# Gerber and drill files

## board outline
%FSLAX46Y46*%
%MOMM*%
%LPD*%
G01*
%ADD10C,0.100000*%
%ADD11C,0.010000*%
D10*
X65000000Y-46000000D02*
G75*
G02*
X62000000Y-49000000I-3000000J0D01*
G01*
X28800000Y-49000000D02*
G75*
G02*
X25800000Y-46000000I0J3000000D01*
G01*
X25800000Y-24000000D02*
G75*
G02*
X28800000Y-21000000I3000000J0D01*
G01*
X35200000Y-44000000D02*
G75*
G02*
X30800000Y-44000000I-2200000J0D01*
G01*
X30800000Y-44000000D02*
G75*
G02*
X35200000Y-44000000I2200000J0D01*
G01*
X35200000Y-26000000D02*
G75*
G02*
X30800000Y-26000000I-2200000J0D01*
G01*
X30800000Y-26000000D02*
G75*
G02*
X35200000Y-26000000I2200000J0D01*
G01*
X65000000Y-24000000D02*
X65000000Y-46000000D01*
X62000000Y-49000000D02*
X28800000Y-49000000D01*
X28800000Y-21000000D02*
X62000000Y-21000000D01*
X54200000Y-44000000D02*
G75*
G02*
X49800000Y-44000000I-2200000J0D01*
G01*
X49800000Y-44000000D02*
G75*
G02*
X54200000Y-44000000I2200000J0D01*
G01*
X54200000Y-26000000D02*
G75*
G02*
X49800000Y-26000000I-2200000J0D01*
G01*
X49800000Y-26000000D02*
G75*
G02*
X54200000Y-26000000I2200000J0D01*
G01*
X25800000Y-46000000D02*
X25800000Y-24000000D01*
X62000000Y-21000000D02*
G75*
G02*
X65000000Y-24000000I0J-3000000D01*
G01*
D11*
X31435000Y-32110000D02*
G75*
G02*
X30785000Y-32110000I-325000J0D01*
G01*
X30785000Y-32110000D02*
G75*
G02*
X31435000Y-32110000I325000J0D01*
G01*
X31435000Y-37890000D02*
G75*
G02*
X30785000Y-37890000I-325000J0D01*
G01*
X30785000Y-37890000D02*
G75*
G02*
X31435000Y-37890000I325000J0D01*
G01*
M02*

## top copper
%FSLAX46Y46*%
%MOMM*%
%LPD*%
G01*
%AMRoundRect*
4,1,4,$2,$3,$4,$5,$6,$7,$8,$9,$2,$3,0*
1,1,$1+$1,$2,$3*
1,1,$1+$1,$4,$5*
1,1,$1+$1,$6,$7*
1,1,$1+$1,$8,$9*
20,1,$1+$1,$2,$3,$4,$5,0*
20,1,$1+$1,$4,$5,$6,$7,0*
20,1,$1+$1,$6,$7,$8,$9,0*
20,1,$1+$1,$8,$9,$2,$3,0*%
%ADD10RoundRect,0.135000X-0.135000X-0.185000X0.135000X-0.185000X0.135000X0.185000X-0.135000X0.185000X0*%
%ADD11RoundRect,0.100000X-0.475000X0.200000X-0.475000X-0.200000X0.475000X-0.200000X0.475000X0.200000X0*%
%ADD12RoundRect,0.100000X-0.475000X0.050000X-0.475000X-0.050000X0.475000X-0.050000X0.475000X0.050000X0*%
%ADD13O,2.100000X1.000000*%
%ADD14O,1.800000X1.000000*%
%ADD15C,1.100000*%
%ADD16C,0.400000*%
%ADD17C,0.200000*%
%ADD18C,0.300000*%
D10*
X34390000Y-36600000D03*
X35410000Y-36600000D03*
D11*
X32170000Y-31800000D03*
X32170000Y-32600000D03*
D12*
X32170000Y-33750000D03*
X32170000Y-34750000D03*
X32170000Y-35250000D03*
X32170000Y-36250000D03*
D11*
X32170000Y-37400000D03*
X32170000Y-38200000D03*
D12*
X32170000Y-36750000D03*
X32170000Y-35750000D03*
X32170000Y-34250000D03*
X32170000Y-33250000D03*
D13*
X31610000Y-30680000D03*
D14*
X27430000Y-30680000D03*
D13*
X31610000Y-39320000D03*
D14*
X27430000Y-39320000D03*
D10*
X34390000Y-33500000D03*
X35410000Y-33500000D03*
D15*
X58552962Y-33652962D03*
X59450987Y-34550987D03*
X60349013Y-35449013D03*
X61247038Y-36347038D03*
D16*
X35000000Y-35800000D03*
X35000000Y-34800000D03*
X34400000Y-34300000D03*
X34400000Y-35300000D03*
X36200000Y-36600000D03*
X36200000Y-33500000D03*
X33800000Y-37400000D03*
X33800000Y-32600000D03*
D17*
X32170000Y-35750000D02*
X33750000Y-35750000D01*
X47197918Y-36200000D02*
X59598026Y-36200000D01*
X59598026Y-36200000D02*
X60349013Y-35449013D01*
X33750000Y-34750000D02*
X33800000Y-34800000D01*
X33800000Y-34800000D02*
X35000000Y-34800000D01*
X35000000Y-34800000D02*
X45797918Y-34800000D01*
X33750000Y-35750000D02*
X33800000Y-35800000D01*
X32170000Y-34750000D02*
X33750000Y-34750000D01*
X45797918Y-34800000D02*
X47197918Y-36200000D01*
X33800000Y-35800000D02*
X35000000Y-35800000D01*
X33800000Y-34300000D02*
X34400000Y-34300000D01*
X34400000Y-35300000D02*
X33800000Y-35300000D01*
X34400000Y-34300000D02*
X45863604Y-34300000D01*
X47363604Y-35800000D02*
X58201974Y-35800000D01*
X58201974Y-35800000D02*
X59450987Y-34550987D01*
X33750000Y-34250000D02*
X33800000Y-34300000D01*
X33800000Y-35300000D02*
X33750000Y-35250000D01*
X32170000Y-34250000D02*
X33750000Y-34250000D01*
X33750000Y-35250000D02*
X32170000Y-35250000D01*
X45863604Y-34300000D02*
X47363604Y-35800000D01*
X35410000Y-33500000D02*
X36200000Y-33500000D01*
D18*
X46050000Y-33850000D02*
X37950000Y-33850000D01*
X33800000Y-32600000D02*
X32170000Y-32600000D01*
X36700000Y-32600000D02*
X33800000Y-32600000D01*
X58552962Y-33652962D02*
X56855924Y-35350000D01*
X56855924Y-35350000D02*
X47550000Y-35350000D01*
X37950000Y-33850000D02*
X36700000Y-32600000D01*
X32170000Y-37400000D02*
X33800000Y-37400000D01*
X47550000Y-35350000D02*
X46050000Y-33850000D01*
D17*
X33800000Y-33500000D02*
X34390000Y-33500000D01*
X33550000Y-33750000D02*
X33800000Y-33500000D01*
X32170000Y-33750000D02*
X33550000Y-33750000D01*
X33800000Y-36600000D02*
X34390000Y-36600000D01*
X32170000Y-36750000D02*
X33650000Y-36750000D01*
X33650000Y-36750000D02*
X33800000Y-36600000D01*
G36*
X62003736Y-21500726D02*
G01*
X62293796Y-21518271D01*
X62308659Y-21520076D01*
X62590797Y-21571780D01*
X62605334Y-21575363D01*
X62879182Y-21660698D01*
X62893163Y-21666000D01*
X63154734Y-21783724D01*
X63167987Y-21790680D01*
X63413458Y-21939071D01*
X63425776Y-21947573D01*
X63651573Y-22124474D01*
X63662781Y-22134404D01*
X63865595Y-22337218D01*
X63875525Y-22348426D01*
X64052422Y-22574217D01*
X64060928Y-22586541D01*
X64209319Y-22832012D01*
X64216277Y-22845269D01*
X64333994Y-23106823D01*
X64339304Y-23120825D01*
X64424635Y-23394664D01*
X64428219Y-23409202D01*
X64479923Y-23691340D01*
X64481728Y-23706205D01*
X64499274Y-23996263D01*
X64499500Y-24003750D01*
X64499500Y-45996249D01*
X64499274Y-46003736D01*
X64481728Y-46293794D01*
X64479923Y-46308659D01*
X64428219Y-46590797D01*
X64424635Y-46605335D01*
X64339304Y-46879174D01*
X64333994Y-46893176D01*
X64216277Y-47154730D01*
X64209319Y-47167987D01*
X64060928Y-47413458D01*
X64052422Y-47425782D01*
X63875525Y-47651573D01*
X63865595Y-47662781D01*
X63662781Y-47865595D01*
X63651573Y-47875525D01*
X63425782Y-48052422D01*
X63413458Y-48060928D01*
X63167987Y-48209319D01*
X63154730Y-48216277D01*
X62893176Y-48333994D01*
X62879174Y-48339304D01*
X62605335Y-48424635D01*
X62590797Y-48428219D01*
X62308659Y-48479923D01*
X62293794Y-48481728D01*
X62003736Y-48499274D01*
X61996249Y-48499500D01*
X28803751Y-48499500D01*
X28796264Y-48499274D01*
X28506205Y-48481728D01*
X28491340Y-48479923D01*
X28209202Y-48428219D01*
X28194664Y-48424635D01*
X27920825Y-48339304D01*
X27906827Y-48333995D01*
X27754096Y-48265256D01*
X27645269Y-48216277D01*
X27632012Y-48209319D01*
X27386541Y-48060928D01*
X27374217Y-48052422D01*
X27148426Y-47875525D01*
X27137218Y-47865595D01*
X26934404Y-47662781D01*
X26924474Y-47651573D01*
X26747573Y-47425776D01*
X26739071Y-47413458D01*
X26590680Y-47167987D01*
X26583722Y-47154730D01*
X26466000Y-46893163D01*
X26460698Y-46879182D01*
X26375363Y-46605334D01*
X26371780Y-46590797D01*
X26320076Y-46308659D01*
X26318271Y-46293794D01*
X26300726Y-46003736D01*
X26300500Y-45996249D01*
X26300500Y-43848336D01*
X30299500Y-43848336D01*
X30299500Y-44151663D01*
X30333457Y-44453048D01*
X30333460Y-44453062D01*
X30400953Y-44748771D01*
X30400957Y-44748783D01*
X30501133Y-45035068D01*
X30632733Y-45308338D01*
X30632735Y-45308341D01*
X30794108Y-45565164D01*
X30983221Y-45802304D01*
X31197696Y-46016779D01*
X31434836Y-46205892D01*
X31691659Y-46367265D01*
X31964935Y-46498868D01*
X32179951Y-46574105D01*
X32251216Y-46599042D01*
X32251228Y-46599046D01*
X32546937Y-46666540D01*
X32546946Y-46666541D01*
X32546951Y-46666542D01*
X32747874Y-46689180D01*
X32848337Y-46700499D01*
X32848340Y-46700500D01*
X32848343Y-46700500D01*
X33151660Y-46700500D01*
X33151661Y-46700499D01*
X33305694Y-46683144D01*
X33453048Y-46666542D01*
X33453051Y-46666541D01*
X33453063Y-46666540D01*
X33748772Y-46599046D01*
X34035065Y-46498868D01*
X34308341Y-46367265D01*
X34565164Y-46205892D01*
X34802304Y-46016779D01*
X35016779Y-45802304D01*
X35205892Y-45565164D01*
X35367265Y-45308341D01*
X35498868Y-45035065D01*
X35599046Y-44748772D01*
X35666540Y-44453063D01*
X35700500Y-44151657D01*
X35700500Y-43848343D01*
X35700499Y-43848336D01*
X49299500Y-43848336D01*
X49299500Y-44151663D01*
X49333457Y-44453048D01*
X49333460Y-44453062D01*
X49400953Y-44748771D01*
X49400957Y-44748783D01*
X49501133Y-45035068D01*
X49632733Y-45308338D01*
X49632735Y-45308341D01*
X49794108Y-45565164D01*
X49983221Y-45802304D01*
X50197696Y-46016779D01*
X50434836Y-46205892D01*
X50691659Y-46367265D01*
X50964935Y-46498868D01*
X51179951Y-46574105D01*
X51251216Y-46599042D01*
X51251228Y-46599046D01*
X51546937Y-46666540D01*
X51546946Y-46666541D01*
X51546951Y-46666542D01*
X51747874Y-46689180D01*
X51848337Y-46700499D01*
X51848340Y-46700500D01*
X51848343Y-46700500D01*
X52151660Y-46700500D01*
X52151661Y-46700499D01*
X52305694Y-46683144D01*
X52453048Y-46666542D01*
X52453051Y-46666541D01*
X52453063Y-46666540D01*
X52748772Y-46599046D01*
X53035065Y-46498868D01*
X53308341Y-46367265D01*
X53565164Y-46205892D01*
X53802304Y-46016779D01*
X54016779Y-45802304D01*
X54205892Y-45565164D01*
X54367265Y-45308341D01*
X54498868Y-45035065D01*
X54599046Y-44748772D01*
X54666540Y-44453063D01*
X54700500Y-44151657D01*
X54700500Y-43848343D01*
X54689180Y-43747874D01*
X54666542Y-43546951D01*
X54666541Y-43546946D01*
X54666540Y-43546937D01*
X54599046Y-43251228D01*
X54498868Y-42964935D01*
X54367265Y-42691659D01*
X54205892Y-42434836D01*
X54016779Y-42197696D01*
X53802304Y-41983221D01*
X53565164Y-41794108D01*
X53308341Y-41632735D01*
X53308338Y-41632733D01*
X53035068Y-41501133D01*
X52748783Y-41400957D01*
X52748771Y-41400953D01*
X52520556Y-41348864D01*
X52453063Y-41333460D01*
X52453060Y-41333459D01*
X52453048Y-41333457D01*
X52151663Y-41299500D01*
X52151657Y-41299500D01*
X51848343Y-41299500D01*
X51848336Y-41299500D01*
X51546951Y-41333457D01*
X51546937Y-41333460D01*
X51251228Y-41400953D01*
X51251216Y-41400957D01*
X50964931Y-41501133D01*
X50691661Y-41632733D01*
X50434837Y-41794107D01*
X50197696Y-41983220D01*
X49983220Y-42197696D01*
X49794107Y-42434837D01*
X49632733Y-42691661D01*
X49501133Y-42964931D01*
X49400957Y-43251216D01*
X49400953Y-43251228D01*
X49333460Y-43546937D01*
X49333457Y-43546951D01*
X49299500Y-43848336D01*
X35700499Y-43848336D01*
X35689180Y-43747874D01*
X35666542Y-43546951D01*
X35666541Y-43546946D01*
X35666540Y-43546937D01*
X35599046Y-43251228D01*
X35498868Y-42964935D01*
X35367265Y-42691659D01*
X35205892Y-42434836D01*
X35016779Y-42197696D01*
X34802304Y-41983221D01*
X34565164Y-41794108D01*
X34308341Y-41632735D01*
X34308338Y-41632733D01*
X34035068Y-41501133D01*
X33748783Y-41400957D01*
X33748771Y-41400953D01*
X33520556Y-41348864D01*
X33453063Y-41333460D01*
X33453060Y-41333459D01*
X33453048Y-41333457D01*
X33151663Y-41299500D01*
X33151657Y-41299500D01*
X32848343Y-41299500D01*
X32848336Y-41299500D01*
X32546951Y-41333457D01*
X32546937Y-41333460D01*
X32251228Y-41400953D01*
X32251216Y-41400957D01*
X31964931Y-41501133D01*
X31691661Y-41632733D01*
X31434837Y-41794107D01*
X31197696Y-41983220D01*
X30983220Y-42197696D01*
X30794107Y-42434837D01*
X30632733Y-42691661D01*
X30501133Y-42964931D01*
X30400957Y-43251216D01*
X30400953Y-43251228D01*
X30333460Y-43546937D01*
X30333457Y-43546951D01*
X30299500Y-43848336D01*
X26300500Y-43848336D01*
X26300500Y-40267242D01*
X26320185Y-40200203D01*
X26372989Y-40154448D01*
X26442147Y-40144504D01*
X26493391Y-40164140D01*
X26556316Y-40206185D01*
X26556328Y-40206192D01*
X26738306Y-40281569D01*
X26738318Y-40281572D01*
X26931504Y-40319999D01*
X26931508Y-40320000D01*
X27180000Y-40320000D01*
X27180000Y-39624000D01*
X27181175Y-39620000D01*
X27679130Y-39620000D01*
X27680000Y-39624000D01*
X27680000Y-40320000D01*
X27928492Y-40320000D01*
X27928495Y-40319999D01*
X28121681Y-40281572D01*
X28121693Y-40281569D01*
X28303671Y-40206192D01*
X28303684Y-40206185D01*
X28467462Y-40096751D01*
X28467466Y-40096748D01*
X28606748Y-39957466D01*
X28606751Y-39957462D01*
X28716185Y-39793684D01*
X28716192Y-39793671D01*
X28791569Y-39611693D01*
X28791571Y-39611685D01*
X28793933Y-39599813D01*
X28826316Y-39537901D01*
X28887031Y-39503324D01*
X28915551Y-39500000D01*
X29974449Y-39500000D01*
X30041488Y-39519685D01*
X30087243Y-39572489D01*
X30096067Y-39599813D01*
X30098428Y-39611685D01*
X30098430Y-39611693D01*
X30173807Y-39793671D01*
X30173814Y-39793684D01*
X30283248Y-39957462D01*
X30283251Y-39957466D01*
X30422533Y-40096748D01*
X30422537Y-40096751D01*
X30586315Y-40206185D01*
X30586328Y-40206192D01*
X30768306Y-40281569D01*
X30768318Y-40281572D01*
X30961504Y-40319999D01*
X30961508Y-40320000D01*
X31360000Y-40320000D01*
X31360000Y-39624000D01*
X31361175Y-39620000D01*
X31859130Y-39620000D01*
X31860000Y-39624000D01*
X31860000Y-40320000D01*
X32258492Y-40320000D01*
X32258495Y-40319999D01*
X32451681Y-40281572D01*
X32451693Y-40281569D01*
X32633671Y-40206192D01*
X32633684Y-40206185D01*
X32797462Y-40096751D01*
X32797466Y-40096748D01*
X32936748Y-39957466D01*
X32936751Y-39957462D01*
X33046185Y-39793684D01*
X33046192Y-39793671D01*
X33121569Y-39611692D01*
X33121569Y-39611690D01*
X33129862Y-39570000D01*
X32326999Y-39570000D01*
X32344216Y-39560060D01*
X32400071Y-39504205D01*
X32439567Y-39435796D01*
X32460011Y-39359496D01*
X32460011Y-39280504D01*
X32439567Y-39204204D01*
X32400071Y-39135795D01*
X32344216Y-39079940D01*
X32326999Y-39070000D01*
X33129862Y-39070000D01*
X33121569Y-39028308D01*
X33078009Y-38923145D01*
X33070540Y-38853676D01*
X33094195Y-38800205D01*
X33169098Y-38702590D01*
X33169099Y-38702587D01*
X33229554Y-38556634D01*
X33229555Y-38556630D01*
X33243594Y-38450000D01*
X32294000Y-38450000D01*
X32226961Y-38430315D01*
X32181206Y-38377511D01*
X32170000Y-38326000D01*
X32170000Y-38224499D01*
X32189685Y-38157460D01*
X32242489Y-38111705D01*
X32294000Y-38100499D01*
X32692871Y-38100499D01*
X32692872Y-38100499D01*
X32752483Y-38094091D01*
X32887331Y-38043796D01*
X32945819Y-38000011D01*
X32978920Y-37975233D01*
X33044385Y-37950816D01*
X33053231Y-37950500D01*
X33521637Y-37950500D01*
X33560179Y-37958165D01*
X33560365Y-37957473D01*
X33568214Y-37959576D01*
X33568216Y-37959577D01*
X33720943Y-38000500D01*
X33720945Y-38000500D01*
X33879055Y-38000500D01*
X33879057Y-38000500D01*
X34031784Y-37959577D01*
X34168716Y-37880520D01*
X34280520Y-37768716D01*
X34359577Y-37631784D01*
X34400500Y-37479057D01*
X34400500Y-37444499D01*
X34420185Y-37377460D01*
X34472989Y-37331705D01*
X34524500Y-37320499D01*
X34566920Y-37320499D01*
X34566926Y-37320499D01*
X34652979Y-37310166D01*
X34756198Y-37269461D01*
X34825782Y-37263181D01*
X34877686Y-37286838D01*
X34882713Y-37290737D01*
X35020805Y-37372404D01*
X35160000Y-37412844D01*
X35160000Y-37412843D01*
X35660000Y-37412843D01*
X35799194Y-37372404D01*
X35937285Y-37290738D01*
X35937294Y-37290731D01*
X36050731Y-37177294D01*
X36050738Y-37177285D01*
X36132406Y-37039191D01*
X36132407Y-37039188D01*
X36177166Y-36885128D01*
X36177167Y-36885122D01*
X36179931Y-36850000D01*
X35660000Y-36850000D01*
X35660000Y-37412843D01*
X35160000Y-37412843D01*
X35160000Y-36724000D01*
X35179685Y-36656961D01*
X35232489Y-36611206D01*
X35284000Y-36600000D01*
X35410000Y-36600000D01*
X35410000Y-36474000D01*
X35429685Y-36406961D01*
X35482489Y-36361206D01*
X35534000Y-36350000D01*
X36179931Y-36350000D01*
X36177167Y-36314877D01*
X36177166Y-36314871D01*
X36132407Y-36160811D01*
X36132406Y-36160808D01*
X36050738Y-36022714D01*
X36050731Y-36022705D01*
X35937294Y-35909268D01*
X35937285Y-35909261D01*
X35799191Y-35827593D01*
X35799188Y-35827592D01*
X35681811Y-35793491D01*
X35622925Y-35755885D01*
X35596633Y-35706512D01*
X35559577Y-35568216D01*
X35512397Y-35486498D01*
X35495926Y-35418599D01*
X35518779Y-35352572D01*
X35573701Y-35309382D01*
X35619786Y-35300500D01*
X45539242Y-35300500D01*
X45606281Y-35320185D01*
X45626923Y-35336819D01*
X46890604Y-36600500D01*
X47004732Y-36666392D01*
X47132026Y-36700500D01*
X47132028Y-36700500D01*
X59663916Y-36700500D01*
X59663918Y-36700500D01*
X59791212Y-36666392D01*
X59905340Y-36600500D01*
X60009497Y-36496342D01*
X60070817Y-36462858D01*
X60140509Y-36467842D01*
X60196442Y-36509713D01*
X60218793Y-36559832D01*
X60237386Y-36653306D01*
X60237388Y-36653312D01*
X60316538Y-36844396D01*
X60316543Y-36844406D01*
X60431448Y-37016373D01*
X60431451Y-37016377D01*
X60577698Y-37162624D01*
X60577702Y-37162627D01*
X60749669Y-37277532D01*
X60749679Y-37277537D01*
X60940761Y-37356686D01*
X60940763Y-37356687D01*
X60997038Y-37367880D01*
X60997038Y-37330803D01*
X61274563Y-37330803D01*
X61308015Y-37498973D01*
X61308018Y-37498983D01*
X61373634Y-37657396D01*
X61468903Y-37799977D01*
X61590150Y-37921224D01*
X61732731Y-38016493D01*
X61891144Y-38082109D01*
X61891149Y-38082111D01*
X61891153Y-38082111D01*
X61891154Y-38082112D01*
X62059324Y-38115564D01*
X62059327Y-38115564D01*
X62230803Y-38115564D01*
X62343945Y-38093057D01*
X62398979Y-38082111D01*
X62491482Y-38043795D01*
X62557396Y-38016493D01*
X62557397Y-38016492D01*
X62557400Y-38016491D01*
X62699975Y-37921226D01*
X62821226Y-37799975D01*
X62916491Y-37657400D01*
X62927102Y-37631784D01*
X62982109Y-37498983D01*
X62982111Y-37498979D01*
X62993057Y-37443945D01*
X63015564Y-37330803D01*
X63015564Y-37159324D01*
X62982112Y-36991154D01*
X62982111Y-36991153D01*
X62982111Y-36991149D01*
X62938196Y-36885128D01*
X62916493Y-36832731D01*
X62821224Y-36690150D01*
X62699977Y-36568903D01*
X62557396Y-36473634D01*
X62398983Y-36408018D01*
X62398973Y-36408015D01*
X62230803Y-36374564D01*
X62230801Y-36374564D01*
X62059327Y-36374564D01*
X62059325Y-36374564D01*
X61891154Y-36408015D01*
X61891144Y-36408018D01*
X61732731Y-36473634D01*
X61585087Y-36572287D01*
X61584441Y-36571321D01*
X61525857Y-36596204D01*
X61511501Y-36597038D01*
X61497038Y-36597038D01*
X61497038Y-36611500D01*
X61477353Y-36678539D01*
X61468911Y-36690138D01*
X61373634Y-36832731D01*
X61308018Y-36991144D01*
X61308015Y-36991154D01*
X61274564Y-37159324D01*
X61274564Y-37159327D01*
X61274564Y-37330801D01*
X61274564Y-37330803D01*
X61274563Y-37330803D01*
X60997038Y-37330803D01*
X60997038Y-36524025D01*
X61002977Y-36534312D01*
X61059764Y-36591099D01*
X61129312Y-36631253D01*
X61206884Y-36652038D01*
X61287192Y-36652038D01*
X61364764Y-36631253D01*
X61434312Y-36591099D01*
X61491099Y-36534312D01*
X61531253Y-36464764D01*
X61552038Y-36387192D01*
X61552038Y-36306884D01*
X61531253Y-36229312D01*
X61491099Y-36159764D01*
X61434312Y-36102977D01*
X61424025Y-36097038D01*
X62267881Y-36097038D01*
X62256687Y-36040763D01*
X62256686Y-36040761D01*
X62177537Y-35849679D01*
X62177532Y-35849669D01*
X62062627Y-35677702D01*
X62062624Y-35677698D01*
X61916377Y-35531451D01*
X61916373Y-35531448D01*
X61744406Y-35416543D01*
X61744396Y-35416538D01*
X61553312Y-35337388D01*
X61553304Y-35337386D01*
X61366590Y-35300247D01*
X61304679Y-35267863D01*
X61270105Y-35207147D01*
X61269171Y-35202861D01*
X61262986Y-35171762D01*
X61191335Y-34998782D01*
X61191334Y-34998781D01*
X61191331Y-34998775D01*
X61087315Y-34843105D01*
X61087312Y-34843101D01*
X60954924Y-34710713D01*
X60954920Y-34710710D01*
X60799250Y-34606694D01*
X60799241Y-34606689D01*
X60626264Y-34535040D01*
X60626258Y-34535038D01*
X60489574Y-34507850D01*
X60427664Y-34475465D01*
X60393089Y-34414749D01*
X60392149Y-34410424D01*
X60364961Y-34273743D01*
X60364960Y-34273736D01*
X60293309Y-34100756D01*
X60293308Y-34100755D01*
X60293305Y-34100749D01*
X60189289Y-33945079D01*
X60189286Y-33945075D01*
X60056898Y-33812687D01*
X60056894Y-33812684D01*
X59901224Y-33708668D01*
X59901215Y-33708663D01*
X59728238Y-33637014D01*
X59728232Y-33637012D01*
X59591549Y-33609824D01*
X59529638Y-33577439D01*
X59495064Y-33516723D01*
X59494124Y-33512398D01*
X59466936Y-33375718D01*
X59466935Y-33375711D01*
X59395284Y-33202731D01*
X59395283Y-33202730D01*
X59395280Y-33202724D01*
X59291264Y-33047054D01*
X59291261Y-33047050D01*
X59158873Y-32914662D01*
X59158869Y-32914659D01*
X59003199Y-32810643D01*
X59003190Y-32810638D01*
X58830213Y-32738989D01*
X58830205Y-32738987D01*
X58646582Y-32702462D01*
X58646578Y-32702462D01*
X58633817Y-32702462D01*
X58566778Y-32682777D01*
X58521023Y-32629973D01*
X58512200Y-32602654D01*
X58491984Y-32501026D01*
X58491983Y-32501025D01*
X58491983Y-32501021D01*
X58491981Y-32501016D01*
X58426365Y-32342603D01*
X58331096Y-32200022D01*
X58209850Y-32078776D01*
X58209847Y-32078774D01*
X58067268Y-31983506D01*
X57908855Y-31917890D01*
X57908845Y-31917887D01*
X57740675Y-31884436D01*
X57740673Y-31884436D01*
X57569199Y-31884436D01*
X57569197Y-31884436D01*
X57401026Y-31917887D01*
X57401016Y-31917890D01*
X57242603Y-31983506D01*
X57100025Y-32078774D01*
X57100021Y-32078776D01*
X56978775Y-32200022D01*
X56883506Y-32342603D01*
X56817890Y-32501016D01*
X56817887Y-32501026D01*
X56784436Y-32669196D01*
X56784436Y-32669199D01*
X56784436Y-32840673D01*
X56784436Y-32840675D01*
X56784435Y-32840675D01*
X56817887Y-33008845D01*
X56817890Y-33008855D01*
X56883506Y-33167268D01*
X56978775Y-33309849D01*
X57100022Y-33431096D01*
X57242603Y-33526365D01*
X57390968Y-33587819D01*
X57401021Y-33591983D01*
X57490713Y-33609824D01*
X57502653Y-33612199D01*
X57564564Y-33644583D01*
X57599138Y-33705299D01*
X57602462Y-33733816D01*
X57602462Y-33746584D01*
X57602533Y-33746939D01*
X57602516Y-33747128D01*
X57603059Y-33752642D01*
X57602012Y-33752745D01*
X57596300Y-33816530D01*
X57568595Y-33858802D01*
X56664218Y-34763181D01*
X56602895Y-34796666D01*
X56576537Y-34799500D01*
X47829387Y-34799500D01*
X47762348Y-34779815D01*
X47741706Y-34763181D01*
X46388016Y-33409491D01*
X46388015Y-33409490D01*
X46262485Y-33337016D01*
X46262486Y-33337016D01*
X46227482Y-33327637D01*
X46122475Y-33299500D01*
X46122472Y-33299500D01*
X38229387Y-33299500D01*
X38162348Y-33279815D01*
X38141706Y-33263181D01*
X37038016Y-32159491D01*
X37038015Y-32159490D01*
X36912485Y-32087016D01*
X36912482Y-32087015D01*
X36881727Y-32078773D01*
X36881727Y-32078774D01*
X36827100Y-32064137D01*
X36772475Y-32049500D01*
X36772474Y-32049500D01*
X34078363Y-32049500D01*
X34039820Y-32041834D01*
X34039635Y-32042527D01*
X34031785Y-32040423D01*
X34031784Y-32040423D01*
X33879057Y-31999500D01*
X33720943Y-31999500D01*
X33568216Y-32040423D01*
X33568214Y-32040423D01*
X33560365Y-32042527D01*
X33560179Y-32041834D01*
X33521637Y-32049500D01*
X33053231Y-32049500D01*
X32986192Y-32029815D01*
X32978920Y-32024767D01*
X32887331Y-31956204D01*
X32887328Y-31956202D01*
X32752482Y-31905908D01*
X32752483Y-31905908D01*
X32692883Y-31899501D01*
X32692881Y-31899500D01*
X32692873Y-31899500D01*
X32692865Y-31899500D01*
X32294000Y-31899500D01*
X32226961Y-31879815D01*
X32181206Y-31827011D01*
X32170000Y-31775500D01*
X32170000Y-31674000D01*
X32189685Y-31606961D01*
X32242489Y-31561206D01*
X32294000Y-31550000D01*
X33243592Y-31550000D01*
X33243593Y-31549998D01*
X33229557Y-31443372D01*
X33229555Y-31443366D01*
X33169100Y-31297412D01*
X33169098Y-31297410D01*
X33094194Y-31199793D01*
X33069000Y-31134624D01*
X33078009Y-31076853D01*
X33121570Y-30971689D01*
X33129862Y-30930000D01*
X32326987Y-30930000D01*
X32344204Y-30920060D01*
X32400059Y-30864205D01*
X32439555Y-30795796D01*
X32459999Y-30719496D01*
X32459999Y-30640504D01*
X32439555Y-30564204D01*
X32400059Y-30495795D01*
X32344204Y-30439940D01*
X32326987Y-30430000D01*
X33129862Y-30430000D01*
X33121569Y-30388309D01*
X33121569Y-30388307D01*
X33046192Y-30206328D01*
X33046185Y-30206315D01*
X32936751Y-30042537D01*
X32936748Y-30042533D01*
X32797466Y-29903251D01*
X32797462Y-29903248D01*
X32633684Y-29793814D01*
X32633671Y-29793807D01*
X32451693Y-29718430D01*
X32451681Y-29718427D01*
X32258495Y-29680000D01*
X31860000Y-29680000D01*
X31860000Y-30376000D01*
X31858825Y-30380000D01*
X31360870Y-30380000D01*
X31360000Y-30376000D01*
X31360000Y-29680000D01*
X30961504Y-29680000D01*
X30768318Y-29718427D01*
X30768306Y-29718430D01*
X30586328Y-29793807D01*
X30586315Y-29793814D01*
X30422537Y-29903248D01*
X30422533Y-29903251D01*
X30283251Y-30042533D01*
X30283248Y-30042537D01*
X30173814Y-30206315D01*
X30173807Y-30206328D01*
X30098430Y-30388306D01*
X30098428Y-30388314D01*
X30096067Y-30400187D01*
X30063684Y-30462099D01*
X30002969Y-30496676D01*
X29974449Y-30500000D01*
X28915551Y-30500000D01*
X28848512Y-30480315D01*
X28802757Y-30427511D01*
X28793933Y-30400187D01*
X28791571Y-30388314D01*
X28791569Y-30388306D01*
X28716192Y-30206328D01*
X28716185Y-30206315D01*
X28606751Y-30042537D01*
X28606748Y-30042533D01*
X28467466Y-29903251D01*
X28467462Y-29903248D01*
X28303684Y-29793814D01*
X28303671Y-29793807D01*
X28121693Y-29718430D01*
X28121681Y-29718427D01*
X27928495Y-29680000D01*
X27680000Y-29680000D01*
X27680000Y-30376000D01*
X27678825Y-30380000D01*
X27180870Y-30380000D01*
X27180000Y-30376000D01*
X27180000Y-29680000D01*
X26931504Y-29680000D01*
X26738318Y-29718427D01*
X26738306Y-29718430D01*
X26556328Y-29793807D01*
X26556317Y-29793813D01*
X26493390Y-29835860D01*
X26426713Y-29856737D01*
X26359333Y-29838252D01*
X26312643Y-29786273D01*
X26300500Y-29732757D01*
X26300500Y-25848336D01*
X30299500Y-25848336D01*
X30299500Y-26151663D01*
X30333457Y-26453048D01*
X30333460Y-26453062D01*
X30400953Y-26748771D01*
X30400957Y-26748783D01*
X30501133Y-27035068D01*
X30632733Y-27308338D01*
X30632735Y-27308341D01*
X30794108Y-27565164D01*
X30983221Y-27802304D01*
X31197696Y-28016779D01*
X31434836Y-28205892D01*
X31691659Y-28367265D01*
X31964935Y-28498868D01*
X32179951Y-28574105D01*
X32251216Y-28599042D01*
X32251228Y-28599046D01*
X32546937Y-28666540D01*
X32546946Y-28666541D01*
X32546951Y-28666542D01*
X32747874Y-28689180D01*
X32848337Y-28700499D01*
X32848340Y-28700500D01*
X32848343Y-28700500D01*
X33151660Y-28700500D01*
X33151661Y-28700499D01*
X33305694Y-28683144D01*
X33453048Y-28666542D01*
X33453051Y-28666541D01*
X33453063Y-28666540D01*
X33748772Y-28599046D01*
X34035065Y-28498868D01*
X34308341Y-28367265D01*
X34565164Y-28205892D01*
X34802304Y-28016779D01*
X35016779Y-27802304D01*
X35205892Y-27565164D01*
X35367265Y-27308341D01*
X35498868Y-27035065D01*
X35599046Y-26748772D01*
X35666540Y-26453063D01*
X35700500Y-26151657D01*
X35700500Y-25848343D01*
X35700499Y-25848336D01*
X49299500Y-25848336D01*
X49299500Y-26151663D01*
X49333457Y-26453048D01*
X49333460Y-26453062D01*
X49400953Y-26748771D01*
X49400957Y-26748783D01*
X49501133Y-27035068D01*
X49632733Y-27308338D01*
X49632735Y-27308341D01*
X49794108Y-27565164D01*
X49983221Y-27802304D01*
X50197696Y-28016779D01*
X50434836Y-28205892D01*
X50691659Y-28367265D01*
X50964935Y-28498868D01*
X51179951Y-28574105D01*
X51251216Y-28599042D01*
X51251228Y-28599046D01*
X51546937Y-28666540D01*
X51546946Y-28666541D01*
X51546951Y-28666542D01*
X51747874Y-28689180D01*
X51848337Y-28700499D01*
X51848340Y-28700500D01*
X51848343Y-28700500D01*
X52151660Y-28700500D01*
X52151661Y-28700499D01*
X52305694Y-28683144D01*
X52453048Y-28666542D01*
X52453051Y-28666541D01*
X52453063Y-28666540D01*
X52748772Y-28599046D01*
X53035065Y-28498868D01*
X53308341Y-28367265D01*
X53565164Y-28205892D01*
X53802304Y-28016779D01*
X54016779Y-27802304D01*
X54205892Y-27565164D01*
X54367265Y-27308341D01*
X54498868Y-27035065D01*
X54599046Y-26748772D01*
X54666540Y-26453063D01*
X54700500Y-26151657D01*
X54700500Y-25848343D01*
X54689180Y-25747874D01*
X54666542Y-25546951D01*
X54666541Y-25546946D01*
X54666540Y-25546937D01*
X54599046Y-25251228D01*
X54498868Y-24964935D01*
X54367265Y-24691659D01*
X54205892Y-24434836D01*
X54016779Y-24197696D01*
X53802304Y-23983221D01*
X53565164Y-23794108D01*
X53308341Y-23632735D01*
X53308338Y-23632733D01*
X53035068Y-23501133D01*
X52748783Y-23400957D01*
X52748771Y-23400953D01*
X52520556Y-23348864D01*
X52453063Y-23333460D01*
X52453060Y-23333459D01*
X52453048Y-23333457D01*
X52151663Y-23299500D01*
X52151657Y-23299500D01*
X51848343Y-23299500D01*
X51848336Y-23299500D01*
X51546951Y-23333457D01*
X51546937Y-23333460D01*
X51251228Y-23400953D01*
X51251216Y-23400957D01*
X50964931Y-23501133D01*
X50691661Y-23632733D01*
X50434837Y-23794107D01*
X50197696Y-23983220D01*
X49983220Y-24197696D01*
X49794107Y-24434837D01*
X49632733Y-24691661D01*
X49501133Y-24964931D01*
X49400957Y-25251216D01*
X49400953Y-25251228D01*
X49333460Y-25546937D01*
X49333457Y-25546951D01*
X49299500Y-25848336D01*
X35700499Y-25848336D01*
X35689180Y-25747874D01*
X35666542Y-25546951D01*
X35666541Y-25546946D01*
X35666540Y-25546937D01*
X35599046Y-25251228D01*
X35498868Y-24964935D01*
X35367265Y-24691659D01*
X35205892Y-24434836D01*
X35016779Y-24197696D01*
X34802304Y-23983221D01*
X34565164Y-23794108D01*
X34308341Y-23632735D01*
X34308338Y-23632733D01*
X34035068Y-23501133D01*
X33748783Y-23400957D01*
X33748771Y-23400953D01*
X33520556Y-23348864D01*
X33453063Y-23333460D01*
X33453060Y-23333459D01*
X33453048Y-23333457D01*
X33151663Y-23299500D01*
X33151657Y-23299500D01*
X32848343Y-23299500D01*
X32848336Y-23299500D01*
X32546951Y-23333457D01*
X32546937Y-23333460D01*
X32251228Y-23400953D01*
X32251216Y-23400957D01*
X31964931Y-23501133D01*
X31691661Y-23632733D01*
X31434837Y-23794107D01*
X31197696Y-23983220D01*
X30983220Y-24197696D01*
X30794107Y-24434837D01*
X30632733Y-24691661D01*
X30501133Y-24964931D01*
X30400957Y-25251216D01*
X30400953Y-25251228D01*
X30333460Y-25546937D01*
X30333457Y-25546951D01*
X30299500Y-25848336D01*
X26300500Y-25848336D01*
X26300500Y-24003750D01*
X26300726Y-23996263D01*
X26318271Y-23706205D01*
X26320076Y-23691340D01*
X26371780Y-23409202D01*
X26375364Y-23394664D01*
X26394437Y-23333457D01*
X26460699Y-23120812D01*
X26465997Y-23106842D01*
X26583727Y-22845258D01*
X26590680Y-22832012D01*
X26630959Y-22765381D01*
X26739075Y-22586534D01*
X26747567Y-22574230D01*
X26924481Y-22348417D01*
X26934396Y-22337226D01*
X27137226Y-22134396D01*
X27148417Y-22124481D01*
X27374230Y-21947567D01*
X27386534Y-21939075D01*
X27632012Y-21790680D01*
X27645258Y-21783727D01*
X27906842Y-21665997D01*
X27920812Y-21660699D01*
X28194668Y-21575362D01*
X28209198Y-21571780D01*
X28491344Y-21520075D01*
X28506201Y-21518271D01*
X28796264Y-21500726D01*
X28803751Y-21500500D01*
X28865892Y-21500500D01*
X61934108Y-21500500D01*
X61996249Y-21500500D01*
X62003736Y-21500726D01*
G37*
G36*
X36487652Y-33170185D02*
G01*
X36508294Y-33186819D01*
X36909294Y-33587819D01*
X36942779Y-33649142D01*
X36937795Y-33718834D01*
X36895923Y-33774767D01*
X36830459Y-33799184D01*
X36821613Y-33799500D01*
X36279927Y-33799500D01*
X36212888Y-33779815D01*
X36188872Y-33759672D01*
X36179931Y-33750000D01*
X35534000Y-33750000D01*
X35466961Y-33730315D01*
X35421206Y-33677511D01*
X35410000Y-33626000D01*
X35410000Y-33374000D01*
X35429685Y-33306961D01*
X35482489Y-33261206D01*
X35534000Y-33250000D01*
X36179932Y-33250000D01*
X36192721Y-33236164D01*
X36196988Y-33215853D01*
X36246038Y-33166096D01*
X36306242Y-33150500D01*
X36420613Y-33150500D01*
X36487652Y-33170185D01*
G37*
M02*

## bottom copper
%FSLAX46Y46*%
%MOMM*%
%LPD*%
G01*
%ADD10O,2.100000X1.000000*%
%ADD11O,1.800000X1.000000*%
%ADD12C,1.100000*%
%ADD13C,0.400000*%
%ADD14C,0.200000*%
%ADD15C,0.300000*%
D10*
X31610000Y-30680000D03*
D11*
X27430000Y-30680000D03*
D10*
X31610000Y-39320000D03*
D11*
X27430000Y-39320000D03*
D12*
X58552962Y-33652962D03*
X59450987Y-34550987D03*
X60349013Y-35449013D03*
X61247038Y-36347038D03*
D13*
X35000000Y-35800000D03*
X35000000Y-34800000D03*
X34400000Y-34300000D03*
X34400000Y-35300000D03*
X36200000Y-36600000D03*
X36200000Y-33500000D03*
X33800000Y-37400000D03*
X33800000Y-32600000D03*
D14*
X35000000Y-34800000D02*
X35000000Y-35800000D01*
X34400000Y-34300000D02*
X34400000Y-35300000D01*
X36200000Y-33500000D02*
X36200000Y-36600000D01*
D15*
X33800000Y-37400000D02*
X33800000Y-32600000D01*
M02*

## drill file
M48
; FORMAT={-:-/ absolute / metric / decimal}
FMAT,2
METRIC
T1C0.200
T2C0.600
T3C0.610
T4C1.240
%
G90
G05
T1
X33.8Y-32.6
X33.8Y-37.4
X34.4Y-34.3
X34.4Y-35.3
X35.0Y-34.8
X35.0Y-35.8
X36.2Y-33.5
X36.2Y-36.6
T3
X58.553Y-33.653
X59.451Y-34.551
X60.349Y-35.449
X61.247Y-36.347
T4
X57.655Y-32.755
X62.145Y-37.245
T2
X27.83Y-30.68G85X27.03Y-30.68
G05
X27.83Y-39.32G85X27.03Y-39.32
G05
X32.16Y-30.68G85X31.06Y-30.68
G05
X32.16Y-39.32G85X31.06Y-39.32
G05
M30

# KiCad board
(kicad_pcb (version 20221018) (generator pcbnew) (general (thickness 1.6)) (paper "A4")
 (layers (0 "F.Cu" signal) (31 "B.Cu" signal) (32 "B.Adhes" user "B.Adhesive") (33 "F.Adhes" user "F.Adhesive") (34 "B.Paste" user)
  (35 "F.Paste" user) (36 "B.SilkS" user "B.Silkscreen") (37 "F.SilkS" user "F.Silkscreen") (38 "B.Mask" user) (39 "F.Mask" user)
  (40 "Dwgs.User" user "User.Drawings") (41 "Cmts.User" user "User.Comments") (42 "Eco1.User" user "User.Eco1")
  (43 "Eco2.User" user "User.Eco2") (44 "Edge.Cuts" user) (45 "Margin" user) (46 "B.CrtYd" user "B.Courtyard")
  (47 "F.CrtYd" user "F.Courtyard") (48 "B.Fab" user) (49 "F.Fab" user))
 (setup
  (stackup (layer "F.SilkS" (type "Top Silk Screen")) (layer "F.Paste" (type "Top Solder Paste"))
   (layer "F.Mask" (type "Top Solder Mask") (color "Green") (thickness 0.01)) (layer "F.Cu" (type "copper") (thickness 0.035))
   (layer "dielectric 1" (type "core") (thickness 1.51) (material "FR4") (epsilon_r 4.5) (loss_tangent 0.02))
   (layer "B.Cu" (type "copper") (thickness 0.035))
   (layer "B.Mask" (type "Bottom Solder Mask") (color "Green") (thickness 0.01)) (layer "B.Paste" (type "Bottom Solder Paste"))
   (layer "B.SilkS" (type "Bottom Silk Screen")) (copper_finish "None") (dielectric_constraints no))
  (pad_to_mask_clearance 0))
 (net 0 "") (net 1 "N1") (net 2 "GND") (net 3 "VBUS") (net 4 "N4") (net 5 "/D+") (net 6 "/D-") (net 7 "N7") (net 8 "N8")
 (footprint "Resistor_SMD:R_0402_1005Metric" (layer "F.Cu") (at 34.9 36.6)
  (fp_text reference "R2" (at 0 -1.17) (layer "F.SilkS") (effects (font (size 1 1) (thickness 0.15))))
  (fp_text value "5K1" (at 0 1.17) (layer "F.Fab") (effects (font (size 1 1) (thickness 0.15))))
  (pad "1" smd roundrect (at -0.51 0) (size 0.54 0.64) (layers "F.Cu" "F.Paste" "F.Mask") (roundrect_rratio 0.25) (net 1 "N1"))
  (pad "2" smd roundrect (at 0.51 0) (size 0.54 0.64) (layers "F.Cu" "F.Paste" "F.Mask") (roundrect_rratio 0.25) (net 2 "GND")))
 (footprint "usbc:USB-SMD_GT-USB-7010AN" (layer "F.Cu") (at 29.8 35 -90)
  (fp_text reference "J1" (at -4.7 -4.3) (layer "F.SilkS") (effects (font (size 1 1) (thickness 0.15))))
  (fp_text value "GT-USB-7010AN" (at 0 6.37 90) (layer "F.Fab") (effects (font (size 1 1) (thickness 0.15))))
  (fp_circle (center -2.89 -1.31) (end -2.565 -1.31) (stroke (width 0.01) (type default)) (fill none) (layer "Edge.Cuts"))
  (fp_circle (center 2.89 -1.31) (end 3.215 -1.31) (stroke (width 0.01) (type default)) (fill none) (layer "Edge.Cuts"))
  (pad "A1" smd roundrect (at -3.2 -2.37 270) (size 0.6 1.15) (layers "F.Cu" "F.Paste" "F.Mask") (roundrect_rratio 0.1666666667)
   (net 2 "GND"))
  (pad "A4" smd roundrect (at -2.4 -2.37 270) (size 0.6 1.15) (layers "F.Cu" "F.Paste" "F.Mask") (roundrect_rratio 0.1666666667)
   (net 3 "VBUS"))
  (pad "A5" smd roundrect (at -1.25 -2.37 270) (size 0.3 1.15) (layers "F.Cu" "F.Paste" "F.Mask") (roundrect_rratio 0.3333333333)
   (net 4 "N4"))
  (pad "A6" smd roundrect (at -0.25 -2.37 270) (size 0.3 1.15) (layers "F.Cu" "F.Paste" "F.Mask") (roundrect_rratio 0.3333333333)
   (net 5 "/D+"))
  (pad "A7" smd roundrect (at 0.25 -2.37 270) (size 0.3 1.15) (layers "F.Cu" "F.Paste" "F.Mask") (roundrect_rratio 0.3333333333)
   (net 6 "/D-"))
  (pad "A8" smd roundrect (at 1.25 -2.37 270) (size 0.3 1.15) (layers "F.Cu" "F.Paste" "F.Mask") (roundrect_rratio 0.3333333333)
   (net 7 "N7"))
  (pad "A9" smd roundrect (at 2.4 -2.37 270) (size 0.6 1.15) (layers "F.Cu" "F.Paste" "F.Mask") (roundrect_rratio 0.1666666667)
   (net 3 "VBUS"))
  (pad "A12" smd roundrect (at 3.2 -2.37 270) (size 0.6 1.15) (layers "F.Cu" "F.Paste" "F.Mask") (roundrect_rratio 0.1666666667)
   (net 2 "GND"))
  (pad "B5" smd roundrect (at 1.75 -2.37 270) (size 0.3 1.15) (layers "F.Cu" "F.Paste" "F.Mask") (roundrect_rratio 0.3333333333)
   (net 1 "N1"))
  (pad "B6" smd roundrect (at 0.75 -2.37 270) (size 0.3 1.15) (layers "F.Cu" "F.Paste" "F.Mask") (roundrect_rratio 0.3333333333)
   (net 5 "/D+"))
  (pad "B7" smd roundrect (at -0.75 -2.37 270) (size 0.3 1.15) (layers "F.Cu" "F.Paste" "F.Mask") (roundrect_rratio 0.3333333333)
   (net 6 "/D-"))
  (pad "B8" smd roundrect (at -1.75 -2.37 270) (size 0.3 1.15) (layers "F.Cu" "F.Paste" "F.Mask") (roundrect_rratio 0.3333333333)
   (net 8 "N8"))
  (pad "S1" thru_hole oval (at -4.32 -1.81 270) (size 1 2.1) (drill oval 0.599999 1.699997) (layers "*.Cu" "*.Mask") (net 2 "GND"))
  (pad "S1" thru_hole oval (at -4.32 2.37 270) (size 1 1.8) (drill oval 0.599999 1.399997) (layers "*.Cu" "*.Mask") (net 2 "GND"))
  (pad "S1" thru_hole oval (at 4.32 -1.81 270) (size 1 2.1) (drill oval 0.599999 1.700022) (layers "*.Cu" "*.Mask") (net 2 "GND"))
  (pad "S1" thru_hole oval (at 4.32 2.37 270) (size 1 1.8) (drill oval 0.599999 1.399997) (layers "*.Cu" "*.Mask") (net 2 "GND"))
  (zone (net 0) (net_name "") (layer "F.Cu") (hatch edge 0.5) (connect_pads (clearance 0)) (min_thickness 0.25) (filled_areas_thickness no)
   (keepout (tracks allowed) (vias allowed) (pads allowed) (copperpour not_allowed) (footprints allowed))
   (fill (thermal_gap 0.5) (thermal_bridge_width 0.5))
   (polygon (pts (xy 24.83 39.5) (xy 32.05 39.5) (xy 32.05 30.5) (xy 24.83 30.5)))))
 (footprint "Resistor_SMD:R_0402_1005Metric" (layer "F.Cu") (at 34.9 33.5)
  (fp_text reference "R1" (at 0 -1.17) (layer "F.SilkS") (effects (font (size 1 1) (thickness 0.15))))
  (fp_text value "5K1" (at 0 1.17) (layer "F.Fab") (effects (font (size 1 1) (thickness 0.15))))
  (pad "1" smd roundrect (at -0.51 0) (size 0.54 0.64) (layers "F.Cu" "F.Paste" "F.Mask") (roundrect_rratio 0.25) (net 4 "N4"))
  (pad "2" smd roundrect (at 0.51 0) (size 0.54 0.64) (layers "F.Cu" "F.Paste" "F.Mask") (roundrect_rratio 0.25) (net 2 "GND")))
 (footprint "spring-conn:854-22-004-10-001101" (layer "F.Cu") (at 59.9 35 -45)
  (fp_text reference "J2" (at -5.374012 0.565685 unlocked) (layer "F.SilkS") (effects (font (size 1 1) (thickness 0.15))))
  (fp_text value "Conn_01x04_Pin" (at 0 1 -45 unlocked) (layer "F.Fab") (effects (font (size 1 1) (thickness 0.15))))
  (pad "" np_thru_hole circle (at -3.175 0 315) (size 1.24 1.24) (drill 1.24) (layers "*.Cu" "*.Mask"))
  (pad "" np_thru_hole circle (at 3.175 0 315) (size 1.24 1.24) (drill 1.24) (layers "*.Cu" "*.Mask"))
  (pad "1" thru_hole circle (at -1.905 0 315) (size 1.1 1.1) (drill 0.61) (layers "*.Cu" "*.Mask") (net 3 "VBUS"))
  (pad "2" thru_hole circle (at -0.635 0 315) (size 1.1 1.1) (drill 0.61) (layers "*.Cu" "*.Mask") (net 6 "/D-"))
  (pad "3" thru_hole circle (at 0.635 0 315) (size 1.1 1.1) (drill 0.61) (layers "*.Cu" "*.Mask") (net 5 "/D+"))
  (pad "4" thru_hole circle (at 1.905 0 315) (size 1.1 1.1) (drill 0.61) (layers "*.Cu" "*.Mask") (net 2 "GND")))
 (gr_arc (start 65 46) (mid 64.12132 48.12132) (end 62 49) (stroke (width 0.1) (type default)) (layer "Edge.Cuts"))
 (gr_arc (start 28.8 49) (mid 26.67868 48.12132) (end 25.8 46) (stroke (width 0.1) (type default)) (layer "Edge.Cuts"))
 (gr_arc (start 25.8 24) (mid 26.67868 21.87868) (end 28.8 21) (stroke (width 0.1) (type default)) (layer "Edge.Cuts"))
 (gr_circle (center 33 44) (end 35.2 44) (stroke (width 0.1) (type default)) (fill none) (layer "Edge.Cuts"))
 (gr_circle (center 33 26) (end 35.2 26) (stroke (width 0.1) (type default)) (fill none) (layer "Edge.Cuts"))
 (gr_line (start 65 24) (end 65 46) (stroke (width 0.1) (type default)) (layer "Edge.Cuts"))
 (gr_line (start 62 49) (end 28.8 49) (stroke (width 0.1) (type default)) (layer "Edge.Cuts"))
 (gr_line (start 28.8 21) (end 62 21) (stroke (width 0.1) (type default)) (layer "Edge.Cuts"))
 (gr_circle (center 52 44) (end 54.2 44) (stroke (width 0.1) (type default)) (fill none) (layer "Edge.Cuts"))
 (gr_circle (center 52 26) (end 54.2 26) (stroke (width 0.1) (type default)) (fill none) (layer "Edge.Cuts"))
 (gr_line (start 25.8 46) (end 25.8 24) (stroke (width 0.1) (type default)) (layer "Edge.Cuts"))
 (gr_arc (start 62 21) (mid 64.12132 21.87868) (end 65 24) (stroke (width 0.1) (type default)) (layer "Edge.Cuts"))
 (segment (start 32.17 35.75) (end 33.75 35.75) (width 0.2) (layer "F.Cu") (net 5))
 (segment (start 47.197918 36.2) (end 59.598026 36.2) (width 0.2) (layer "F.Cu") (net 5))
 (segment (start 59.598026 36.2) (end 60.349013 35.449013) (width 0.2) (layer "F.Cu") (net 5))
 (segment (start 33.75 34.75) (end 33.8 34.8) (width 0.2) (layer "F.Cu") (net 5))
 (segment (start 33.8 34.8) (end 35 34.8) (width 0.2) (layer "F.Cu") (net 5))
 (segment (start 35 34.8) (end 45.797918 34.8) (width 0.2) (layer "F.Cu") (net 5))
 (segment (start 33.75 35.75) (end 33.8 35.8) (width 0.2) (layer "F.Cu") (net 5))
 (segment (start 32.17 34.75) (end 33.75 34.75) (width 0.2) (layer "F.Cu") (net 5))
 (segment (start 45.797918 34.8) (end 47.197918 36.2) (width 0.2) (layer "F.Cu") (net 5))
 (segment (start 33.8 35.8) (end 35 35.8) (width 0.2) (layer "F.Cu") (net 5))
 (via (at 35 35.8) (size 0.4) (drill 0.2) (layers "F.Cu" "B.Cu") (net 5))
 (via (at 35 34.8) (size 0.4) (drill 0.2) (layers "F.Cu" "B.Cu") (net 5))
 (segment (start 35 34.8) (end 35 35.8) (width 0.2) (layer "B.Cu") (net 5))
 (segment (start 33.8 34.3) (end 34.4 34.3) (width 0.2) (layer "F.Cu") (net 6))
 (segment (start 34.4 35.3) (end 33.8 35.3) (width 0.2) (layer "F.Cu") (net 6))
 (segment (start 34.4 34.3) (end 45.863604 34.3) (width 0.2) (layer "F.Cu") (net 6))
 (segment (start 47.363604 35.8) (end 58.201974 35.8) (width 0.2) (layer "F.Cu") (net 6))
 (segment (start 58.201974 35.8) (end 59.450987 34.550987) (width 0.2) (layer "F.Cu") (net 6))
 (segment (start 33.75 34.25) (end 33.8 34.3) (width 0.2) (layer "F.Cu") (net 6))
 (segment (start 33.8 35.3) (end 33.75 35.25) (width 0.2) (layer "F.Cu") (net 6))
 (segment (start 32.17 34.25) (end 33.75 34.25) (width 0.2) (layer "F.Cu") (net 6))
 (segment (start 33.75 35.25) (end 32.17 35.25) (width 0.2) (layer "F.Cu") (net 6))
 (segment (start 45.863604 34.3) (end 47.363604 35.8) (width 0.2) (layer "F.Cu") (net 6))
 (via (at 34.4 34.3) (size 0.4) (drill 0.2) (layers "F.Cu" "B.Cu") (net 6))
 (via (at 34.4 35.3) (size 0.4) (drill 0.2) (layers "F.Cu" "B.Cu") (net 6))
 (segment (start 34.4 34.3) (end 34.4 35.3) (width 0.2) (layer "B.Cu") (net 6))
 (segment (start 35.41 33.5) (end 36.2 33.5) (width 0.2) (layer "F.Cu") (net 2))
 (via (at 36.2 36.6) (size 0.4) (drill 0.2) (layers "F.Cu" "B.Cu") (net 2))
 (via (at 36.2 33.5) (size 0.4) (drill 0.2) (layers "F.Cu" "B.Cu") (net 2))
 (segment (start 36.2 33.5) (end 36.2 36.6) (width 0.2) (layer "B.Cu") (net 2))
 (segment (start 46.05 33.85) (end 37.95 33.85) (width 0.3) (layer "F.Cu") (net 3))
 (segment (start 33.8 32.6) (end 32.17 32.6) (width 0.3) (layer "F.Cu") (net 3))
 (segment (start 36.7 32.6) (end 33.8 32.6) (width 0.3) (layer "F.Cu") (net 3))
 (segment (start 58.552962 33.652962) (end 56.855924 35.35) (width 0.3) (layer "F.Cu") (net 3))
 (segment (start 56.855924 35.35) (end 47.55 35.35) (width 0.3) (layer "F.Cu") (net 3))
 (segment (start 37.95 33.85) (end 36.7 32.6) (width 0.3) (layer "F.Cu") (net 3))
 (segment (start 32.17 37.4) (end 33.8 37.4) (width 0.3) (layer "F.Cu") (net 3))
 (segment (start 47.55 35.35) (end 46.05 33.85) (width 0.3) (layer "F.Cu") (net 3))
 (via (at 33.8 37.4) (size 0.4) (drill 0.2) (layers "F.Cu" "B.Cu") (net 3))
 (via (at 33.8 32.6) (size 0.4) (drill 0.2) (layers "F.Cu" "B.Cu") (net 3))
 (segment (start 33.8 37.4) (end 33.8 32.6) (width 0.3) (layer "B.Cu") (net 3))
 (segment (start 33.8 33.5) (end 34.39 33.5) (width 0.2) (layer "F.Cu") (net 4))
 (segment (start 33.55 33.75) (end 33.8 33.5) (width 0.2) (layer "F.Cu") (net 4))
 (segment (start 32.17 33.75) (end 33.55 33.75) (width 0.2) (layer "F.Cu") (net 4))
 (segment (start 33.8 36.6) (end 34.39 36.6) (width 0.2) (layer "F.Cu") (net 1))
 (segment (start 32.17 36.75) (end 33.65 36.75) (width 0.2) (layer "F.Cu") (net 1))
 (segment (start 33.65 36.75) (end 33.8 36.6) (width 0.2) (layer "F.Cu") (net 1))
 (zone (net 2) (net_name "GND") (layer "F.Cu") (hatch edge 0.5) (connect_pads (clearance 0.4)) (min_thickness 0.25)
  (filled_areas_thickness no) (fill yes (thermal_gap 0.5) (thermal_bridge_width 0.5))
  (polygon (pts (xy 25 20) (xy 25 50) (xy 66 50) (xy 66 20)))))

